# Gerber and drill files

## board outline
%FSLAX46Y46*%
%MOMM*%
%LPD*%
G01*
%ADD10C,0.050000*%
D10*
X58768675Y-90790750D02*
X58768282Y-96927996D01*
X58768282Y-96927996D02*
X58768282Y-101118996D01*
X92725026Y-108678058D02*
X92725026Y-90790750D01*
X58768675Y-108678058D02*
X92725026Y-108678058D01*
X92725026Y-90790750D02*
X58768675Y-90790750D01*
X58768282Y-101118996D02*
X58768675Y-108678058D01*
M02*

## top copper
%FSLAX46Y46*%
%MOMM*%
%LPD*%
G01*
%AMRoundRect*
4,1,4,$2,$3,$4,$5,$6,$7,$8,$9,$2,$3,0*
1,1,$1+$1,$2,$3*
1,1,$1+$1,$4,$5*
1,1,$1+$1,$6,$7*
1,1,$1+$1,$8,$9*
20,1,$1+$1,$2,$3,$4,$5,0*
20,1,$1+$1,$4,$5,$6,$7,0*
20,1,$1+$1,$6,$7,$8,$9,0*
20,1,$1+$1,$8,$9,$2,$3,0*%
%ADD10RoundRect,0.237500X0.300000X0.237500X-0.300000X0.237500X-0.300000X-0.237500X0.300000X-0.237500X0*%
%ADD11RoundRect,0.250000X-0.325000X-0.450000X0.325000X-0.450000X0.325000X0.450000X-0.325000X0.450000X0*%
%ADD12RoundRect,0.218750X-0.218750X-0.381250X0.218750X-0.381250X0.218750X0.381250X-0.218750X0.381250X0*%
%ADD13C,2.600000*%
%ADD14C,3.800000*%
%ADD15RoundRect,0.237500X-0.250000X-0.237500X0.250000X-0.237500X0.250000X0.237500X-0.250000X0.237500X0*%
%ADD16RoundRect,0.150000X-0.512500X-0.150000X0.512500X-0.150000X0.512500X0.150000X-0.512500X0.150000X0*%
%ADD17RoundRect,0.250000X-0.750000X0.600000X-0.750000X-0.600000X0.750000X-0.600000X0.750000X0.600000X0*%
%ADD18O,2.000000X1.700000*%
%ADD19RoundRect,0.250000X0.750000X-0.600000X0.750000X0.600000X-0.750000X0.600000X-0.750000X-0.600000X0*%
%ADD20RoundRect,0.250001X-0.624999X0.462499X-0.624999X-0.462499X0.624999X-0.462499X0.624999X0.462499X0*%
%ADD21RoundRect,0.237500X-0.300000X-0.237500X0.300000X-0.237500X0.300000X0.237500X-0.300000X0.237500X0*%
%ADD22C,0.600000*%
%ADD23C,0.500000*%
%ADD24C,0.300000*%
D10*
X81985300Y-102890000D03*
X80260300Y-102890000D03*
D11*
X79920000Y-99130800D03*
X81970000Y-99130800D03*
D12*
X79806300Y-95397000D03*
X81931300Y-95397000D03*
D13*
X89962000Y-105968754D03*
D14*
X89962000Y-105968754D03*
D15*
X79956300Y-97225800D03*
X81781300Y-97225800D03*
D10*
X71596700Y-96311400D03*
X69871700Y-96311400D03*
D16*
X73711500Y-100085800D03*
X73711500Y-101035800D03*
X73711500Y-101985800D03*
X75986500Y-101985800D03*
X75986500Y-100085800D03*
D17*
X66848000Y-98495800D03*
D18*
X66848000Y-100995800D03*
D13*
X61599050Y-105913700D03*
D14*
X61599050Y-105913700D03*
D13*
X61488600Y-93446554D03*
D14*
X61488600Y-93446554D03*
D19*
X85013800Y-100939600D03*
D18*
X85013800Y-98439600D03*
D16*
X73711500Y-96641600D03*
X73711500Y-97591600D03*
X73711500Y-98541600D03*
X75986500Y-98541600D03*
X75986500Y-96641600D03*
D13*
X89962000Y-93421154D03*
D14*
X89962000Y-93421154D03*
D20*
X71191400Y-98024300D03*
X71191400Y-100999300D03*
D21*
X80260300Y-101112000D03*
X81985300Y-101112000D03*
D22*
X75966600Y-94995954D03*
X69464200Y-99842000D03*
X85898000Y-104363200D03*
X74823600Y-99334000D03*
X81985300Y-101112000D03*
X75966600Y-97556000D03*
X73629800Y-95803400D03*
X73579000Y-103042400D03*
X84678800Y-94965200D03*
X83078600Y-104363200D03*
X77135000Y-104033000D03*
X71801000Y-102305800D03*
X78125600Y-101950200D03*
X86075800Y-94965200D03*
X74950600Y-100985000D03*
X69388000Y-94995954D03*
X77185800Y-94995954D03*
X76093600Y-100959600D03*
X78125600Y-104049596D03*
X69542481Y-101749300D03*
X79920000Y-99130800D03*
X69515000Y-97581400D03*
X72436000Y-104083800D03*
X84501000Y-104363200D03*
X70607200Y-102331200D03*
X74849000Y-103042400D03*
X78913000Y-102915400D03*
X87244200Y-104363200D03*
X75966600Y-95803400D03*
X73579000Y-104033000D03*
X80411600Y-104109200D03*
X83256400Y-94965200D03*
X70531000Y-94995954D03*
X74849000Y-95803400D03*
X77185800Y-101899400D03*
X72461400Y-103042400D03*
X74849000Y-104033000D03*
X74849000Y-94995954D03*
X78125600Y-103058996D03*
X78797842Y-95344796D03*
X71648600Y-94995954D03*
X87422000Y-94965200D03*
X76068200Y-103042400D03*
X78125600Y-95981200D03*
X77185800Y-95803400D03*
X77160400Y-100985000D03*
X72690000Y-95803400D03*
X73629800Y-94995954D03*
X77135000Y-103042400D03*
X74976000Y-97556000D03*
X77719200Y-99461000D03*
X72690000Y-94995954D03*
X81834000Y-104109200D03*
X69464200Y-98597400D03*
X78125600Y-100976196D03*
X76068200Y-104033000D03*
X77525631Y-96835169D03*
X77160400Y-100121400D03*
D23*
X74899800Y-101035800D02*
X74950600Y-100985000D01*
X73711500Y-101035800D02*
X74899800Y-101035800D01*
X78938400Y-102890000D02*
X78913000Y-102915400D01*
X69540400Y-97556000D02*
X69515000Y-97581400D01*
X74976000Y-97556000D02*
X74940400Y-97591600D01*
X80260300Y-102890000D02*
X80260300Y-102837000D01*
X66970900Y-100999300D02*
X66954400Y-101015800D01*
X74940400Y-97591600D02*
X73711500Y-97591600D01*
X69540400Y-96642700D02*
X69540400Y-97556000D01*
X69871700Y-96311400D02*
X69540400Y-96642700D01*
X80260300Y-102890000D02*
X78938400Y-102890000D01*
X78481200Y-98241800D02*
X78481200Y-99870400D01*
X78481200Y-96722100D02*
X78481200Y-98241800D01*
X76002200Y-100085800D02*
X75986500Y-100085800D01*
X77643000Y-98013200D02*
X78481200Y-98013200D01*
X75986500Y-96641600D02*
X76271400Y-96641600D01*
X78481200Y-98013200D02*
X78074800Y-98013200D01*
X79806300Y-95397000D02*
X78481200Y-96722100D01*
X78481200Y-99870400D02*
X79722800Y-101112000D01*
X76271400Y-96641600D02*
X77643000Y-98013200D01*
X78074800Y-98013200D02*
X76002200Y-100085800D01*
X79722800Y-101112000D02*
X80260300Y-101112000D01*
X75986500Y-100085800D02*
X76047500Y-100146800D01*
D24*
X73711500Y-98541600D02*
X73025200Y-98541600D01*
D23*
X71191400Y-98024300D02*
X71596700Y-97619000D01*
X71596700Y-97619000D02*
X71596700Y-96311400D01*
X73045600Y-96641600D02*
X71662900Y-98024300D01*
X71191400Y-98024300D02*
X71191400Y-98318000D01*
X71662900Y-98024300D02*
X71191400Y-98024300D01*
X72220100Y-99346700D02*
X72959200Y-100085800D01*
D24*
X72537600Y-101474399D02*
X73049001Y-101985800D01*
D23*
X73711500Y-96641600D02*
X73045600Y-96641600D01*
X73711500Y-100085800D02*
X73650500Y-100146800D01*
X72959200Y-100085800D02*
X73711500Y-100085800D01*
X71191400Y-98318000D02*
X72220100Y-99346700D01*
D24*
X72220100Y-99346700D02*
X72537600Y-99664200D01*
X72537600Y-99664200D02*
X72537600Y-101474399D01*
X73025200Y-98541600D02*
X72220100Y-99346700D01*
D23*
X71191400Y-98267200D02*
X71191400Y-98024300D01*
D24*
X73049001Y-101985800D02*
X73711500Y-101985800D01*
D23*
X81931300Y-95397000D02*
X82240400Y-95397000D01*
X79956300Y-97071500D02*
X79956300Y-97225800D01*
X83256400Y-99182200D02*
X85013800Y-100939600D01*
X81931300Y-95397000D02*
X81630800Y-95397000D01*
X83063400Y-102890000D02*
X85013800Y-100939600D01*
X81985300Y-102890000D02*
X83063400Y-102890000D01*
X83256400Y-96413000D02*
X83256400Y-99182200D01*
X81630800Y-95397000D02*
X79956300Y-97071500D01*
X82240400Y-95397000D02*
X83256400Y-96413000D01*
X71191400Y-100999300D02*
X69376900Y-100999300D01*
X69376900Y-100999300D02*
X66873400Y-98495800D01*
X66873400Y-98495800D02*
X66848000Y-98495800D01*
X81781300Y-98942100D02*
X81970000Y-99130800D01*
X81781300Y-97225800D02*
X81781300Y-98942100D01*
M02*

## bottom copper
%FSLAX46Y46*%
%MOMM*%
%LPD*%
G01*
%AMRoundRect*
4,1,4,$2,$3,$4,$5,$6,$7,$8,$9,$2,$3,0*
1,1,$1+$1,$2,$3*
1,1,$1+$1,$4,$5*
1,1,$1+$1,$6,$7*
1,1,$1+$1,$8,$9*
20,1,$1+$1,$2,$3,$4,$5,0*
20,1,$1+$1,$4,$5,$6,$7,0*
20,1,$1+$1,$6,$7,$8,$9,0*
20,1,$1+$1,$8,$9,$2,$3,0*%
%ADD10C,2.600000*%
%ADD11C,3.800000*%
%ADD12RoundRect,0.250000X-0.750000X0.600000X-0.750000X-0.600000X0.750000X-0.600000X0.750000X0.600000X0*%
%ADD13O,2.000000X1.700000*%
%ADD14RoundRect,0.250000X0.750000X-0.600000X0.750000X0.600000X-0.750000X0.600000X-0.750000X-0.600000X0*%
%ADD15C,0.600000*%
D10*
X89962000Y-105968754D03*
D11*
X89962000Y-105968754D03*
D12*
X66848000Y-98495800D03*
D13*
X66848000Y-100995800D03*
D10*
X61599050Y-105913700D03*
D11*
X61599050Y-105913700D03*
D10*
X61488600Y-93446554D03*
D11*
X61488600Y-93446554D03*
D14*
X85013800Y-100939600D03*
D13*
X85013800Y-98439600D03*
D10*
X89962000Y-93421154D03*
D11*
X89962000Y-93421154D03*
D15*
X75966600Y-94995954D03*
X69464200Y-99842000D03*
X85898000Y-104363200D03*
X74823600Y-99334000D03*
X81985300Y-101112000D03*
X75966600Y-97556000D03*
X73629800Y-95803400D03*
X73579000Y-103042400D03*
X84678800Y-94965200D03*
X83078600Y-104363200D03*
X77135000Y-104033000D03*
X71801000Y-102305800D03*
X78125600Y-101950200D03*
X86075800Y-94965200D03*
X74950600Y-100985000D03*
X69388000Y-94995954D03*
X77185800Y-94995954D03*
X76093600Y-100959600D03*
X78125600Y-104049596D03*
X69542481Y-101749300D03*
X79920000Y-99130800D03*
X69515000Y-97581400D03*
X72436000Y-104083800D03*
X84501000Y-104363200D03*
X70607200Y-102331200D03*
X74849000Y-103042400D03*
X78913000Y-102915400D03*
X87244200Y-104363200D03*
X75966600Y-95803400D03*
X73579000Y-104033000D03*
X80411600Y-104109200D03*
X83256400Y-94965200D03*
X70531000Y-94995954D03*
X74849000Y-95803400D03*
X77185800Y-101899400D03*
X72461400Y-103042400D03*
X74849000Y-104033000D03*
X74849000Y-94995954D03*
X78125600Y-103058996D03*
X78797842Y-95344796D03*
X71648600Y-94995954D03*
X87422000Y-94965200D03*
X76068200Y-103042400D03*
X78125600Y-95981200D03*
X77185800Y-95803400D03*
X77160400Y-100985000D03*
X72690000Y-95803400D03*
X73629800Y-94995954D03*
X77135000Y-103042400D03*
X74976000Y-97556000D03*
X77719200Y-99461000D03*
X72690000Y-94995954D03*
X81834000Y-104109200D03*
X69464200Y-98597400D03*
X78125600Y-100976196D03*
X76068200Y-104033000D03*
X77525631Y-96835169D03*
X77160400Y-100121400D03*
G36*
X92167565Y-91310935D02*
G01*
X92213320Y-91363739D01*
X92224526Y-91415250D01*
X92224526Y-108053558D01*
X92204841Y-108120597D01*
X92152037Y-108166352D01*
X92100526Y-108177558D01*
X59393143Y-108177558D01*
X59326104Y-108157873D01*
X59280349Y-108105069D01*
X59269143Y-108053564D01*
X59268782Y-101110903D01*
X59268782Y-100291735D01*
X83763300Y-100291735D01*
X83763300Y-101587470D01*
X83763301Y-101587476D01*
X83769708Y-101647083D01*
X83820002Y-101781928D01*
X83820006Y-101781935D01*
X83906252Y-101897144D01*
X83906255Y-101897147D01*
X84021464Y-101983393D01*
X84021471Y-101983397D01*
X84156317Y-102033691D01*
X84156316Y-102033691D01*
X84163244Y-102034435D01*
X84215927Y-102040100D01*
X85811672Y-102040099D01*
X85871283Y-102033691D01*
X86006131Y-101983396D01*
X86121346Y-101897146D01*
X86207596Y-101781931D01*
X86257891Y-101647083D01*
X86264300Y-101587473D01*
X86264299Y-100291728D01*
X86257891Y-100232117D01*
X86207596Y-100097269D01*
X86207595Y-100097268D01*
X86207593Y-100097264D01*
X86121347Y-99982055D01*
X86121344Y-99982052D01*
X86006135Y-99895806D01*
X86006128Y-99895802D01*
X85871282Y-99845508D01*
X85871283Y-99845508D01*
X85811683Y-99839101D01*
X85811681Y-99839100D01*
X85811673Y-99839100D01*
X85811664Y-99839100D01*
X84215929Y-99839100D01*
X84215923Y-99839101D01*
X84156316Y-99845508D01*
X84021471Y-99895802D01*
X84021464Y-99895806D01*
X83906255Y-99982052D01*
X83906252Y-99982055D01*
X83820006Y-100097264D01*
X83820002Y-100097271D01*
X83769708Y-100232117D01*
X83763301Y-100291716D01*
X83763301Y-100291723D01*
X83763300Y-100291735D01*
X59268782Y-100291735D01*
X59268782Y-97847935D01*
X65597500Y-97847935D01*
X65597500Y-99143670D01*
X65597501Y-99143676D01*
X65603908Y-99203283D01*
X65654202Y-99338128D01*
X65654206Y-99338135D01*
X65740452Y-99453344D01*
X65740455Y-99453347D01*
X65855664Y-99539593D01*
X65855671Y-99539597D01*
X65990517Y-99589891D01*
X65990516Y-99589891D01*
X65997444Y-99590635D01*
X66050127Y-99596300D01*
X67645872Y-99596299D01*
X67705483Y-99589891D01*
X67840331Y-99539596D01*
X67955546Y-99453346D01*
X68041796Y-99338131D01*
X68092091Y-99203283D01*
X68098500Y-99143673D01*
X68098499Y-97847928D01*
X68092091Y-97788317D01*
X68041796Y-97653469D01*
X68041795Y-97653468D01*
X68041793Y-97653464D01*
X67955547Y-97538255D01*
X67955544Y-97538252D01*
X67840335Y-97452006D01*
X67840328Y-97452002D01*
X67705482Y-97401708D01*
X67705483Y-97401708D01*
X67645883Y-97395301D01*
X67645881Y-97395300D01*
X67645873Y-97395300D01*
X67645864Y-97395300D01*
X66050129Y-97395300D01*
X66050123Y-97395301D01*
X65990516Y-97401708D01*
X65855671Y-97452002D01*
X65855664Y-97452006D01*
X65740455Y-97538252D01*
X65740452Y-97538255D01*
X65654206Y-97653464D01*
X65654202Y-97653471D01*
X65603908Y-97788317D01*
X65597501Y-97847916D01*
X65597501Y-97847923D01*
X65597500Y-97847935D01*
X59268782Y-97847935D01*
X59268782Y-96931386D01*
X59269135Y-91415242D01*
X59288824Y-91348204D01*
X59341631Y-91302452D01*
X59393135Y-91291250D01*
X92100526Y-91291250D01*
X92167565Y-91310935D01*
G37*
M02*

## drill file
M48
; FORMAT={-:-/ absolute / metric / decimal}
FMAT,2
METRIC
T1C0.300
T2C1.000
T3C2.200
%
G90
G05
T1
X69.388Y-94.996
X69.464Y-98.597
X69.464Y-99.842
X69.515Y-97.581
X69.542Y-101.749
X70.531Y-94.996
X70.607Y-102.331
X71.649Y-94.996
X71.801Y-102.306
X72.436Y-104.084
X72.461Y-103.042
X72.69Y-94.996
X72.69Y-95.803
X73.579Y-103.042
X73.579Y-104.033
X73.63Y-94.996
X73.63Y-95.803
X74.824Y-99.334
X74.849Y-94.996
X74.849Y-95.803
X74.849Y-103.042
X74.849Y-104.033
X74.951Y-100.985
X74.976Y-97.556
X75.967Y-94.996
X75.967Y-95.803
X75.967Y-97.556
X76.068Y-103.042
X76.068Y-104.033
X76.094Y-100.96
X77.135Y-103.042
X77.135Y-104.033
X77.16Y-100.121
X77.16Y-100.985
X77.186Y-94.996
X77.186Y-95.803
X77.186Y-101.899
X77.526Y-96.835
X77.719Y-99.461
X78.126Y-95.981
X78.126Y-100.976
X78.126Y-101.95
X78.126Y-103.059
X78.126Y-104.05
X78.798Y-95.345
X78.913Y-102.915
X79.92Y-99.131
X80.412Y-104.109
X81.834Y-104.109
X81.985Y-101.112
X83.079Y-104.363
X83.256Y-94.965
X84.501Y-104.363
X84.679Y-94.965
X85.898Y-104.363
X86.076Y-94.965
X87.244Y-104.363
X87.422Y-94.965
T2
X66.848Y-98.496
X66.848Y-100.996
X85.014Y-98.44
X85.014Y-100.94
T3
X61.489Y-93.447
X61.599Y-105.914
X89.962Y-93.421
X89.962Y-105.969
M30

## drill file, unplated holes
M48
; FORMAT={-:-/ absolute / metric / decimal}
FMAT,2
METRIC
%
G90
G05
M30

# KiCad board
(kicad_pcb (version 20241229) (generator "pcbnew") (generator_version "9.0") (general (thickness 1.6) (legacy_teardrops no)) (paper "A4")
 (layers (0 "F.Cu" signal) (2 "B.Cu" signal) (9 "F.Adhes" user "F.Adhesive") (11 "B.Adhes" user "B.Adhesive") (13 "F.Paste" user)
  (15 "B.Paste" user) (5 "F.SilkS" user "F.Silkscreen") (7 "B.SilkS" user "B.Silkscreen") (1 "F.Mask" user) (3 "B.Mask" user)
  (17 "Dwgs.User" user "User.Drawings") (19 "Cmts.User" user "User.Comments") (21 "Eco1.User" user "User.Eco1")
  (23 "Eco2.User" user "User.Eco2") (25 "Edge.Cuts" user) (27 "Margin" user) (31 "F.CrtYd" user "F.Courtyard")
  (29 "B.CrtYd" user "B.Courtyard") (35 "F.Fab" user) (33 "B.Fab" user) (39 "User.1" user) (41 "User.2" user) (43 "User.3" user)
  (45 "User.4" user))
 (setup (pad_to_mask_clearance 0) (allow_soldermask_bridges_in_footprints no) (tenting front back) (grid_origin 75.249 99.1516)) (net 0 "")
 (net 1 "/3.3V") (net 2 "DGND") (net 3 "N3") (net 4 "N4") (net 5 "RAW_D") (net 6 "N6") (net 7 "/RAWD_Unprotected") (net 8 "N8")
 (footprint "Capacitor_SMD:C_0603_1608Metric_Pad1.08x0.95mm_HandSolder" (layer "F.Cu") (at 81.1228 102.89 180)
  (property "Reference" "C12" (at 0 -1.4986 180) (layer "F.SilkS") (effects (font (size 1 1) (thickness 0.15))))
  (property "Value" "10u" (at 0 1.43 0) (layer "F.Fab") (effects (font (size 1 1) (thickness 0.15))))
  (pad "1" smd roundrect (at -0.8625 0 180) (size 1.075 0.95) (layers "F.Cu" "F.Mask" "F.Paste") (roundrect_rratio 0.25) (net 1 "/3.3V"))
  (pad "2" smd roundrect (at 0.8625 0 180) (size 1.075 0.95) (layers "F.Cu" "F.Mask" "F.Paste") (roundrect_rratio 0.25) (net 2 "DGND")))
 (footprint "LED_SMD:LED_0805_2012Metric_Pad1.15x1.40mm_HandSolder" (layer "F.Cu") (at 80.945 99.1308)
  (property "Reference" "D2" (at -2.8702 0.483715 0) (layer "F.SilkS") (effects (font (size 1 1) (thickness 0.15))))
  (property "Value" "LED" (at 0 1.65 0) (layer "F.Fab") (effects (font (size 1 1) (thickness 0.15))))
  (pad "1" smd roundrect (at -1.025 0) (size 1.15 1.4) (layers "F.Cu" "F.Mask" "F.Paste") (roundrect_rratio 0.217391) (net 2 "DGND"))
  (pad "2" smd roundrect (at 1.025 0) (size 1.15 1.4) (layers "F.Cu" "F.Mask" "F.Paste") (roundrect_rratio 0.217391) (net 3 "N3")))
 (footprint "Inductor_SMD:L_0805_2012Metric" (layer "F.Cu") (at 80.8688 95.397)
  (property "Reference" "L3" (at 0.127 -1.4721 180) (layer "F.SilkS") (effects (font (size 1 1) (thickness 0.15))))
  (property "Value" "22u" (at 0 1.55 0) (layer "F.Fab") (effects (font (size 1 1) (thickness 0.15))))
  (pad "1" smd roundrect (at -1.0625 0) (size 0.875 1.2) (layers "F.Cu" "F.Mask" "F.Paste") (roundrect_rratio 0.25) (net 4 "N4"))
  (pad "2" smd roundrect (at 1.0625 0) (size 0.875 1.2) (layers "F.Cu" "F.Mask" "F.Paste") (roundrect_rratio 0.25) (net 1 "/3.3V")))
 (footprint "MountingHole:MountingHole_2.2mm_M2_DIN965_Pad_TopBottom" (layer "F.Cu") (at 89.962 105.968754)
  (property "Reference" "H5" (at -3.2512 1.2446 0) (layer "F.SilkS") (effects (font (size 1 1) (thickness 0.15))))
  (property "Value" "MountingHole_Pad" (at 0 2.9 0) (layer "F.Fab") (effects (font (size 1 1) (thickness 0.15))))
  (pad "1" thru_hole circle (at 0 0) (size 2.6 2.6) (drill 2.2) (layers "*.Cu" "*.Mask") (remove_unused_layers no) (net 2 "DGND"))
  (pad "1" connect circle (at 0 0) (size 3.8 3.8) (layers "F.Cu" "F.Mask") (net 2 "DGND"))
  (pad "1" connect circle (at 0 0) (size 3.8 3.8) (layers "B.Cu" "B.Mask") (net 2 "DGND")))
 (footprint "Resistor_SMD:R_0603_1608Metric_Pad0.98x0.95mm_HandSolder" (layer "F.Cu") (at 80.8688 97.2258)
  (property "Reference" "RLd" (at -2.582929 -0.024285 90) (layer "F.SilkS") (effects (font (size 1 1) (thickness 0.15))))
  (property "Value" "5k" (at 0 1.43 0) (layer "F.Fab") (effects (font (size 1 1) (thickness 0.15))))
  (pad "1" smd roundrect (at -0.9125 0) (size 0.975 0.95) (layers "F.Cu" "F.Mask" "F.Paste") (roundrect_rratio 0.25) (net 1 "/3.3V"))
  (pad "2" smd roundrect (at 0.9125 0) (size 0.975 0.95) (layers "F.Cu" "F.Mask" "F.Paste") (roundrect_rratio 0.25) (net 3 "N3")))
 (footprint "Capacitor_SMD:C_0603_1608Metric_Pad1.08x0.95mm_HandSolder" (layer "F.Cu") (at 70.7342 96.3114 180)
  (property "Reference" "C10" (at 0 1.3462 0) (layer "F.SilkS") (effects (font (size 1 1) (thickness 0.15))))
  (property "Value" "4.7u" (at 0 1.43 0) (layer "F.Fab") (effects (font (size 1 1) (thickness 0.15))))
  (pad "1" smd roundrect (at -0.8625 0 180) (size 1.075 0.95) (layers "F.Cu" "F.Mask" "F.Paste") (roundrect_rratio 0.25) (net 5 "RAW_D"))
  (pad "2" smd roundrect (at 0.8625 0 180) (size 1.075 0.95) (layers "F.Cu" "F.Mask" "F.Paste") (roundrect_rratio 0.25) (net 2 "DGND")))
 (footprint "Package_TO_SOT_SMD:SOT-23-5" (layer "F.Cu") (at 74.849 101.0358)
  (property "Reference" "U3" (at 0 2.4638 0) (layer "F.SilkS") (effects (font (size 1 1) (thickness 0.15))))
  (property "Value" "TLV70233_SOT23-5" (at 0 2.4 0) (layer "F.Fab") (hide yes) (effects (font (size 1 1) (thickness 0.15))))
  (pad "1" smd roundrect (at -1.1375 -0.95) (size 1.325 0.6) (layers "F.Cu" "F.Mask" "F.Paste") (roundrect_rratio 0.25) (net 5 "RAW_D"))
  (pad "2" smd roundrect (at -1.1375 0) (size 1.325 0.6) (layers "F.Cu" "F.Mask" "F.Paste") (roundrect_rratio 0.25) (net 2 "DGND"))
  (pad "3" smd roundrect (at -1.1375 0.95) (size 1.325 0.6) (layers "F.Cu" "F.Mask" "F.Paste") (roundrect_rratio 0.25) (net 5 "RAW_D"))
  (pad "4" smd roundrect (at 1.1375 0.95) (size 1.325 0.6) (layers "F.Cu" "F.Mask" "F.Paste") (roundrect_rratio 0.25) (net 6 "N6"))
  (pad "5" smd roundrect (at 1.1375 -0.95) (size 1.325 0.6) (layers "F.Cu" "F.Mask" "F.Paste") (roundrect_rratio 0.25) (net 4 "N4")))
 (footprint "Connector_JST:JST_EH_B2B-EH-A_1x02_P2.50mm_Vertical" (layer "F.Cu") (at 66.848 98.4958 -90)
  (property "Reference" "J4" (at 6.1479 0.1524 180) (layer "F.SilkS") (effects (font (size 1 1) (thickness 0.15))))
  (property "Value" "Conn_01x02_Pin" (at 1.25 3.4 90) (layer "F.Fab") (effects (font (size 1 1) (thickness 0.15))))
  (pad "1" thru_hole roundrect (at 0 0 270) (size 1.7 2) (drill 1) (layers "*.Cu" "*.Mask") (remove_unused_layers no)
   (roundrect_rratio 0.147059) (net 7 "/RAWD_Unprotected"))
  (pad "2" thru_hole oval (at 2.5 0 270) (size 1.7 2) (drill 1) (layers "*.Cu" "*.Mask") (remove_unused_layers no) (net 2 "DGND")))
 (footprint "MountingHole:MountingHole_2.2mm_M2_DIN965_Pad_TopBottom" (layer "F.Cu") (at 61.59905 105.9137)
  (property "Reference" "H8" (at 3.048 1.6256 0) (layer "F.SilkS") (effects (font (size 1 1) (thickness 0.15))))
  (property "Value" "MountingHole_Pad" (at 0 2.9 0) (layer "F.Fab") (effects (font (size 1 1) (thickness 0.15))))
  (pad "1" thru_hole circle (at 0 0) (size 2.6 2.6) (drill 2.2) (layers "*.Cu" "*.Mask") (remove_unused_layers no) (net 2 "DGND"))
  (pad "1" connect circle (at 0 0) (size 3.8 3.8) (layers "F.Cu" "F.Mask") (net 2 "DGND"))
  (pad "1" connect circle (at 0 0) (size 3.8 3.8) (layers "B.Cu" "B.Mask") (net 2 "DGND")))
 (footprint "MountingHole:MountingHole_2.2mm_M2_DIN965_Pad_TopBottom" (layer "F.Cu") (at 61.4886 93.446554)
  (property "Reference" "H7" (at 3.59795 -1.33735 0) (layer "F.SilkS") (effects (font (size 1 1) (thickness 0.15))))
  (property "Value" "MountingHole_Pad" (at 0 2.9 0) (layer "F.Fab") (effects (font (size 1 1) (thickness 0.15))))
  (pad "1" thru_hole circle (at 0 0) (size 2.6 2.6) (drill 2.2) (layers "*.Cu" "*.Mask") (remove_unused_layers no) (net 2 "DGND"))
  (pad "1" connect circle (at 0 0) (size 3.8 3.8) (layers "F.Cu" "F.Mask") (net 2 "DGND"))
  (pad "1" connect circle (at 0 0) (size 3.8 3.8) (layers "B.Cu" "B.Mask") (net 2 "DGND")))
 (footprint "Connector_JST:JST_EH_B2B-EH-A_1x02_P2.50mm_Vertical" (layer "F.Cu") (at 85.0138 100.9396 90)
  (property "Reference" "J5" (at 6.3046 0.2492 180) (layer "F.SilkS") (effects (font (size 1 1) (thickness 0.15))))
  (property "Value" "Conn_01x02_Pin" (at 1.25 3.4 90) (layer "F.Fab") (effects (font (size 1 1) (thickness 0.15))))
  (pad "1" thru_hole roundrect (at 0 0 90) (size 1.7 2) (drill 1) (layers "*.Cu" "*.Mask") (remove_unused_layers no)
   (roundrect_rratio 0.147059) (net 1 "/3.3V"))
  (pad "2" thru_hole oval (at 2.5 0 90) (size 1.7 2) (drill 1) (layers "*.Cu" "*.Mask") (remove_unused_layers no) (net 2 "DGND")))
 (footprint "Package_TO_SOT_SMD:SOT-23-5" (layer "F.Cu") (at 74.849 97.5916)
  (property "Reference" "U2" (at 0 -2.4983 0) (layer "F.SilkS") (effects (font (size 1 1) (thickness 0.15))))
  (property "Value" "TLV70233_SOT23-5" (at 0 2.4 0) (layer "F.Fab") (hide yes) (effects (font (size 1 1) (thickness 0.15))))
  (pad "1" smd roundrect (at -1.1375 -0.95) (size 1.325 0.6) (layers "F.Cu" "F.Mask" "F.Paste") (roundrect_rratio 0.25) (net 5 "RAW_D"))
  (pad "2" smd roundrect (at -1.1375 0) (size 1.325 0.6) (layers "F.Cu" "F.Mask" "F.Paste") (roundrect_rratio 0.25) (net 2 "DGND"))
  (pad "3" smd roundrect (at -1.1375 0.95) (size 1.325 0.6) (layers "F.Cu" "F.Mask" "F.Paste") (roundrect_rratio 0.25) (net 5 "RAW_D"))
  (pad "4" smd roundrect (at 1.1375 0.95) (size 1.325 0.6) (layers "F.Cu" "F.Mask" "F.Paste") (roundrect_rratio 0.25) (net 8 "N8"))
  (pad "5" smd roundrect (at 1.1375 -0.95) (size 1.325 0.6) (layers "F.Cu" "F.Mask" "F.Paste") (roundrect_rratio 0.25) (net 4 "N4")))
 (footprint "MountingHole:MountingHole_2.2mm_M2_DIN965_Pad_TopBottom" (layer "F.Cu") (at 89.962 93.421154)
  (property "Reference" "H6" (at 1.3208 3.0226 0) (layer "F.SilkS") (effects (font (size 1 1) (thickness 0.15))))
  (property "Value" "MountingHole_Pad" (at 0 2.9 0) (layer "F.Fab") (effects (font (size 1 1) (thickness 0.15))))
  (pad "1" thru_hole circle (at 0 0) (size 2.6 2.6) (drill 2.2) (layers "*.Cu" "*.Mask") (remove_unused_layers no) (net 2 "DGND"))
  (pad "1" connect circle (at 0 0) (size 3.8 3.8) (layers "F.Cu" "F.Mask") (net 2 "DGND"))
  (pad "1" connect circle (at 0 0) (size 3.8 3.8) (layers "B.Cu" "B.Mask") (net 2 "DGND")))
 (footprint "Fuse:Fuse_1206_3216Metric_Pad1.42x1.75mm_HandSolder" (layer "F.Cu") (at 71.1914 99.5118 -90)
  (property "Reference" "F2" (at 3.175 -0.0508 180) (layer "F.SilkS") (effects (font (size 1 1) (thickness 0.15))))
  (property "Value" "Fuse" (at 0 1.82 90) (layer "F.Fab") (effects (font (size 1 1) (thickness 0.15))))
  (pad "1" smd roundrect (at -1.4875 0 270) (size 1.425 1.75) (layers "F.Cu" "F.Mask" "F.Paste") (roundrect_rratio 0.175439) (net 5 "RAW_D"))
  (pad "2" smd roundrect (at 1.4875 0 270) (size 1.425 1.75) (layers "F.Cu" "F.Mask" "F.Paste") (roundrect_rratio 0.175439)
   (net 7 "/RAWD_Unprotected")))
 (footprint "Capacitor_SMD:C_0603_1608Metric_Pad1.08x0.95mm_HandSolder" (layer "F.Cu") (at 81.1228 101.112)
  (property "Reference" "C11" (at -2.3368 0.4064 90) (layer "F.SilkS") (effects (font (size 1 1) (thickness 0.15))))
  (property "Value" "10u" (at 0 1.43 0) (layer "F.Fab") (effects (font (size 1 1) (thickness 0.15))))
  (pad "1" smd roundrect (at -0.8625 0) (size 1.075 0.95) (layers "F.Cu" "F.Mask" "F.Paste") (roundrect_rratio 0.25) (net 4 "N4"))
  (pad "2" smd roundrect (at 0.8625 0) (size 1.075 0.95) (layers "F.Cu" "F.Mask" "F.Paste") (roundrect_rratio 0.25) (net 2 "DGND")))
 (gr_line (start 58.768675 90.79075) (end 58.768282 96.927996) (stroke (width 0.05) (type default)) (layer "Edge.Cuts"))
 (gr_line (start 58.768282 96.927996) (end 58.768282 101.118996) (stroke (width 0.05) (type default)) (layer "Edge.Cuts"))
 (gr_line (start 92.725026 108.678058) (end 92.725026 90.79075) (stroke (width 0.05) (type default)) (layer "Edge.Cuts"))
 (gr_line (start 58.768675 108.678058) (end 92.725026 108.678058) (stroke (width 0.05) (type default)) (layer "Edge.Cuts"))
 (gr_line (start 92.725026 90.79075) (end 58.768675 90.79075) (stroke (width 0.05) (type default)) (layer "Edge.Cuts"))
 (gr_line (start 58.768282 101.118996) (end 58.768675 108.678058) (stroke (width 0.05) (type default)) (layer "Edge.Cuts"))
 (segment (start 74.8998 101.0358) (end 74.9506 100.985) (width 0.5) (layer "F.Cu") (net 2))
 (segment (start 73.7115 101.0358) (end 74.8998 101.0358) (width 0.5) (layer "F.Cu") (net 2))
 (segment (start 78.9384 102.89) (end 78.913 102.9154) (width 0.5) (layer "F.Cu") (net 2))
 (segment (start 69.5404 97.556) (end 69.515 97.5814) (width 0.5) (layer "F.Cu") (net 2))
 (segment (start 74.976 97.556) (end 74.9404 97.5916) (width 0.5) (layer "F.Cu") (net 2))
 (segment (start 80.2603 102.89) (end 80.2603 102.837) (width 0.5) (layer "F.Cu") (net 2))
 (segment (start 66.9709 100.9993) (end 66.9544 101.0158) (width 0.5) (layer "F.Cu") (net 2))
 (segment (start 74.9404 97.5916) (end 73.7115 97.5916) (width 0.5) (layer "F.Cu") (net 2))
 (segment (start 69.5404 96.6427) (end 69.5404 97.556) (width 0.5) (layer "F.Cu") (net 2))
 (segment (start 69.8717 96.3114) (end 69.5404 96.6427) (width 0.5) (layer "F.Cu") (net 2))
 (segment (start 80.2603 102.89) (end 78.9384 102.89) (width 0.5) (layer "F.Cu") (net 2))
 (via (at 75.9666 94.995954) (size 0.6) (drill 0.3) (layers "F.Cu" "B.Cu") (free yes) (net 2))
 (via (at 69.4642 99.842) (size 0.6) (drill 0.3) (layers "F.Cu" "B.Cu") (free yes) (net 2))
 (via (at 85.898 104.3632) (size 0.6) (drill 0.3) (layers "F.Cu" "B.Cu") (free yes) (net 2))
 (via (at 74.8236 99.334) (size 0.6) (drill 0.3) (layers "F.Cu" "B.Cu") (free yes) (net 2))
 (via (at 81.9853 101.112) (size 0.6) (drill 0.3) (layers "F.Cu" "B.Cu") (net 2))
 (via (at 75.9666 97.556) (size 0.6) (drill 0.3) (layers "F.Cu" "B.Cu") (free yes) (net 2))
 (via (at 73.6298 95.8034) (size 0.6) (drill 0.3) (layers "F.Cu" "B.Cu") (free yes) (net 2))
 (via (at 73.579 103.0424) (size 0.6) (drill 0.3) (layers "F.Cu" "B.Cu") (free yes) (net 2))
 (via (at 84.6788 94.9652) (size 0.6) (drill 0.3) (layers "F.Cu" "B.Cu") (free yes) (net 2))
 (via (at 83.0786 104.3632) (size 0.6) (drill 0.3) (layers "F.Cu" "B.Cu") (free yes) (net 2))
 (via (at 77.135 104.033) (size 0.6) (drill 0.3) (layers "F.Cu" "B.Cu") (free yes) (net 2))
 (via (at 71.801 102.3058) (size 0.6) (drill 0.3) (layers "F.Cu" "B.Cu") (free yes) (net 2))
 (via (at 78.1256 101.9502) (size 0.6) (drill 0.3) (layers "F.Cu" "B.Cu") (free yes) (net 2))
 (via (at 86.0758 94.9652) (size 0.6) (drill 0.3) (layers "F.Cu" "B.Cu") (free yes) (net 2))
 (via (at 74.9506 100.985) (size 0.6) (drill 0.3) (layers "F.Cu" "B.Cu") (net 2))
 (via (at 69.388 94.995954) (size 0.6) (drill 0.3) (layers "F.Cu" "B.Cu") (free yes) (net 2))
 (via (at 77.1858 94.995954) (size 0.6) (drill 0.3) (layers "F.Cu" "B.Cu") (free yes) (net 2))
 (via (at 76.0936 100.9596) (size 0.6) (drill 0.3) (layers "F.Cu" "B.Cu") (free yes) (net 2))
 (via (at 78.1256 104.049596) (size 0.6) (drill 0.3) (layers "F.Cu" "B.Cu") (free yes) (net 2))
 (via (at 69.542481 101.7493) (size 0.6) (drill 0.3) (layers "F.Cu" "B.Cu") (free yes) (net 2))
 (via (at 79.92 99.1308) (size 0.6) (drill 0.3) (layers "F.Cu" "B.Cu") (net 2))
 (via (at 69.515 97.5814) (size 0.6) (drill 0.3) (layers "F.Cu" "B.Cu") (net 2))
 (via (at 72.436 104.0838) (size 0.6) (drill 0.3) (layers "F.Cu" "B.Cu") (free yes) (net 2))
 (via (at 84.501 104.3632) (size 0.6) (drill 0.3) (layers "F.Cu" "B.Cu") (free yes) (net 2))
 (via (at 70.6072 102.3312) (size 0.6) (drill 0.3) (layers "F.Cu" "B.Cu") (free yes) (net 2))
 (via (at 74.849 103.0424) (size 0.6) (drill 0.3) (layers "F.Cu" "B.Cu") (free yes) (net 2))
 (via (at 78.913 102.9154) (size 0.6) (drill 0.3) (layers "F.Cu" "B.Cu") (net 2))
 (via (at 87.2442 104.3632) (size 0.6) (drill 0.3) (layers "F.Cu" "B.Cu") (free yes) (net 2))
 (via (at 75.9666 95.8034) (size 0.6) (drill 0.3) (layers "F.Cu" "B.Cu") (free yes) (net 2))
 (via (at 73.579 104.033) (size 0.6) (drill 0.3) (layers "F.Cu" "B.Cu") (free yes) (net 2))
 (via (at 80.4116 104.1092) (size 0.6) (drill 0.3) (layers "F.Cu" "B.Cu") (free yes) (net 2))
 (via (at 83.2564 94.9652) (size 0.6) (drill 0.3) (layers "F.Cu" "B.Cu") (free yes) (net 2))
 (via (at 70.531 94.995954) (size 0.6) (drill 0.3) (layers "F.Cu" "B.Cu") (free yes) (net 2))
 (via (at 74.849 95.8034) (size 0.6) (drill 0.3) (layers "F.Cu" "B.Cu") (free yes) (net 2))
 (via (at 77.1858 101.8994) (size 0.6) (drill 0.3) (layers "F.Cu" "B.Cu") (free yes) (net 2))
 (via (at 72.4614 103.0424) (size 0.6) (drill 0.3) (layers "F.Cu" "B.Cu") (free yes) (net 2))
 (via (at 74.849 104.033) (size 0.6) (drill 0.3) (layers "F.Cu" "B.Cu") (free yes) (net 2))
 (via (at 74.849 94.995954) (size 0.6) (drill 0.3) (layers "F.Cu" "B.Cu") (free yes) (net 2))
 (via (at 78.1256 103.058996) (size 0.6) (drill 0.3) (layers "F.Cu" "B.Cu") (free yes) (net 2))
 (via (at 78.797842 95.344796) (size 0.6) (drill 0.3) (layers "F.Cu" "B.Cu") (free yes) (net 2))
 (via (at 71.6486 94.995954) (size 0.6) (drill 0.3) (layers "F.Cu" "B.Cu") (free yes) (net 2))
 (via (at 87.422 94.9652) (size 0.6) (drill 0.3) (layers "F.Cu" "B.Cu") (free yes) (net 2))
 (via (at 76.0682 103.0424) (size 0.6) (drill 0.3) (layers "F.Cu" "B.Cu") (free yes) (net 2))
 (via (at 78.1256 95.9812) (size 0.6) (drill 0.3) (layers "F.Cu" "B.Cu") (free yes) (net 2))
 (via (at 77.1858 95.8034) (size 0.6) (drill 0.3) (layers "F.Cu" "B.Cu") (free yes) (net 2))
 (via (at 77.1604 100.985) (size 0.6) (drill 0.3) (layers "F.Cu" "B.Cu") (free yes) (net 2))
 (via (at 72.69 95.8034) (size 0.6) (drill 0.3) (layers "F.Cu" "B.Cu") (free yes) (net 2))
 (via (at 73.6298 94.995954) (size 0.6) (drill 0.3) (layers "F.Cu" "B.Cu") (free yes) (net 2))
 (via (at 77.135 103.0424) (size 0.6) (drill 0.3) (layers "F.Cu" "B.Cu") (free yes) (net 2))
 (via (at 74.976 97.556) (size 0.6) (drill 0.3) (layers "F.Cu" "B.Cu") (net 2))
 (via (at 77.7192 99.461) (size 0.6) (drill 0.3) (layers "F.Cu" "B.Cu") (free yes) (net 2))
 (via (at 72.69 94.995954) (size 0.6) (drill 0.3) (layers "F.Cu" "B.Cu") (free yes) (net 2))
 (via (at 81.834 104.1092) (size 0.6) (drill 0.3) (layers "F.Cu" "B.Cu") (free yes) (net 2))
 (via (at 69.4642 98.5974) (size 0.6) (drill 0.3) (layers "F.Cu" "B.Cu") (free yes) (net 2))
 (via (at 78.1256 100.976196) (size 0.6) (drill 0.3) (layers "F.Cu" "B.Cu") (free yes) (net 2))
 (via (at 76.0682 104.033) (size 0.6) (drill 0.3) (layers "F.Cu" "B.Cu") (free yes) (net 2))
 (via (at 77.525631 96.835169) (size 0.6) (drill 0.3) (layers "F.Cu" "B.Cu") (free yes) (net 2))
 (via (at 77.1604 100.1214) (size 0.6) (drill 0.3) (layers "F.Cu" "B.Cu") (free yes) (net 2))
 (segment (start 78.4812 98.2418) (end 78.4812 99.8704) (width 0.5) (layer "F.Cu") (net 4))
 (segment (start 78.4812 96.7221) (end 78.4812 98.2418) (width 0.5) (layer "F.Cu") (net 4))
 (segment (start 76.0022 100.0858) (end 75.9865 100.0858) (width 0.5) (layer "F.Cu") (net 4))
 (segment (start 77.643 98.0132) (end 78.4812 98.0132) (width 0.5) (layer "F.Cu") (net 4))
 (segment (start 75.9865 96.6416) (end 76.2714 96.6416) (width 0.5) (layer "F.Cu") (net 4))
 (segment (start 78.4812 98.0132) (end 78.0748 98.0132) (width 0.5) (layer "F.Cu") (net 4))
 (segment (start 79.8063 95.397) (end 78.4812 96.7221) (width 0.5) (layer "F.Cu") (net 4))
 (segment (start 78.4812 99.8704) (end 79.7228 101.112) (width 0.5) (layer "F.Cu") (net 4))
 (segment (start 76.2714 96.6416) (end 77.643 98.0132) (width 0.5) (layer "F.Cu") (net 4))
 (segment (start 78.0748 98.0132) (end 76.0022 100.0858) (width 0.5) (layer "F.Cu") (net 4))
 (segment (start 79.7228 101.112) (end 80.2603 101.112) (width 0.5) (layer "F.Cu") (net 4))
 (segment (start 75.9865 100.0858) (end 76.0475 100.1468) (width 0.5) (layer "F.Cu") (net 4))
 (segment (start 73.7115 98.5416) (end 73.0252 98.5416) (width 0.3) (layer "F.Cu") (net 5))
 (segment (start 71.1914 98.0243) (end 71.5967 97.619) (width 0.5) (layer "F.Cu") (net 5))
 (segment (start 71.5967 97.619) (end 71.5967 96.3114) (width 0.5) (layer "F.Cu") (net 5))
 (segment (start 73.0456 96.6416) (end 71.6629 98.0243) (width 0.5) (layer "F.Cu") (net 5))
 (segment (start 71.1914 98.0243) (end 71.1914 98.318) (width 0.5) (layer "F.Cu") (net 5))
 (segment (start 71.6629 98.0243) (end 71.1914 98.0243) (width 0.5) (layer "F.Cu") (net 5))
 (segment (start 72.2201 99.3467) (end 72.9592 100.0858) (width 0.5) (layer "F.Cu") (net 5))
 (segment (start 72.5376 101.474399) (end 73.049001 101.9858) (width 0.3) (layer "F.Cu") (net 5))
 (segment (start 73.7115 96.6416) (end 73.0456 96.6416) (width 0.5) (layer "F.Cu") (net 5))
 (segment (start 73.7115 100.0858) (end 73.6505 100.1468) (width 0.5) (layer "F.Cu") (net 5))
 (segment (start 72.9592 100.0858) (end 73.7115 100.0858) (width 0.5) (layer "F.Cu") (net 5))
 (segment (start 71.1914 98.318) (end 72.2201 99.3467) (width 0.5) (layer "F.Cu") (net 5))
 (segment (start 72.2201 99.3467) (end 72.5376 99.6642) (width 0.3) (layer "F.Cu") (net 5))
 (segment (start 72.5376 99.6642) (end 72.5376 101.474399) (width 0.3) (layer "F.Cu") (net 5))
 (segment (start 73.0252 98.5416) (end 72.2201 99.3467) (width 0.3) (layer "F.Cu") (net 5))
 (segment (start 71.1914 98.2672) (end 71.1914 98.0243) (width 0.5) (layer "F.Cu") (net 5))
 (segment (start 73.049001 101.9858) (end 73.7115 101.9858) (width 0.3) (layer "F.Cu") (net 5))
 (segment (start 81.9313 95.397) (end 82.2404 95.397) (width 0.5) (layer "F.Cu") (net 1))
 (segment (start 79.9563 97.0715) (end 79.9563 97.2258) (width 0.5) (layer "F.Cu") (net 1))
 (segment (start 83.2564 99.1822) (end 85.0138 100.9396) (width 0.5) (layer "F.Cu") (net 1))
 (segment (start 81.9313 95.397) (end 81.6308 95.397) (width 0.5) (layer "F.Cu") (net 1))
 (segment (start 83.0634 102.89) (end 85.0138 100.9396) (width 0.5) (layer "F.Cu") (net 1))
 (segment (start 81.9853 102.89) (end 83.0634 102.89) (width 0.5) (layer "F.Cu") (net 1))
 (segment (start 83.2564 96.413) (end 83.2564 99.1822) (width 0.5) (layer "F.Cu") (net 1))
 (segment (start 81.6308 95.397) (end 79.9563 97.0715) (width 0.5) (layer "F.Cu") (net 1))
 (segment (start 82.2404 95.397) (end 83.2564 96.413) (width 0.5) (layer "F.Cu") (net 1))
 (segment (start 71.1914 100.9993) (end 69.3769 100.9993) (width 0.5) (layer "F.Cu") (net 7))
 (segment (start 69.3769 100.9993) (end 66.8734 98.4958) (width 0.5) (layer "F.Cu") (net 7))
 (segment (start 66.8734 98.4958) (end 66.848 98.4958) (width 0.5) (layer "F.Cu") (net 7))
 (segment (start 81.7813 98.9421) (end 81.97 99.1308) (width 0.5) (layer "F.Cu") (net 3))
 (segment (start 81.7813 97.2258) (end 81.7813 98.9421) (width 0.5) (layer "F.Cu") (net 3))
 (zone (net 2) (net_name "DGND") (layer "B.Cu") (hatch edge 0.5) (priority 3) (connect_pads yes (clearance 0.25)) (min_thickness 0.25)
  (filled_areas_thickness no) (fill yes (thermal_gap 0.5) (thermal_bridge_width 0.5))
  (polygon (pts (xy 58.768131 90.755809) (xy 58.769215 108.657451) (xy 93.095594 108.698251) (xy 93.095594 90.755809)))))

